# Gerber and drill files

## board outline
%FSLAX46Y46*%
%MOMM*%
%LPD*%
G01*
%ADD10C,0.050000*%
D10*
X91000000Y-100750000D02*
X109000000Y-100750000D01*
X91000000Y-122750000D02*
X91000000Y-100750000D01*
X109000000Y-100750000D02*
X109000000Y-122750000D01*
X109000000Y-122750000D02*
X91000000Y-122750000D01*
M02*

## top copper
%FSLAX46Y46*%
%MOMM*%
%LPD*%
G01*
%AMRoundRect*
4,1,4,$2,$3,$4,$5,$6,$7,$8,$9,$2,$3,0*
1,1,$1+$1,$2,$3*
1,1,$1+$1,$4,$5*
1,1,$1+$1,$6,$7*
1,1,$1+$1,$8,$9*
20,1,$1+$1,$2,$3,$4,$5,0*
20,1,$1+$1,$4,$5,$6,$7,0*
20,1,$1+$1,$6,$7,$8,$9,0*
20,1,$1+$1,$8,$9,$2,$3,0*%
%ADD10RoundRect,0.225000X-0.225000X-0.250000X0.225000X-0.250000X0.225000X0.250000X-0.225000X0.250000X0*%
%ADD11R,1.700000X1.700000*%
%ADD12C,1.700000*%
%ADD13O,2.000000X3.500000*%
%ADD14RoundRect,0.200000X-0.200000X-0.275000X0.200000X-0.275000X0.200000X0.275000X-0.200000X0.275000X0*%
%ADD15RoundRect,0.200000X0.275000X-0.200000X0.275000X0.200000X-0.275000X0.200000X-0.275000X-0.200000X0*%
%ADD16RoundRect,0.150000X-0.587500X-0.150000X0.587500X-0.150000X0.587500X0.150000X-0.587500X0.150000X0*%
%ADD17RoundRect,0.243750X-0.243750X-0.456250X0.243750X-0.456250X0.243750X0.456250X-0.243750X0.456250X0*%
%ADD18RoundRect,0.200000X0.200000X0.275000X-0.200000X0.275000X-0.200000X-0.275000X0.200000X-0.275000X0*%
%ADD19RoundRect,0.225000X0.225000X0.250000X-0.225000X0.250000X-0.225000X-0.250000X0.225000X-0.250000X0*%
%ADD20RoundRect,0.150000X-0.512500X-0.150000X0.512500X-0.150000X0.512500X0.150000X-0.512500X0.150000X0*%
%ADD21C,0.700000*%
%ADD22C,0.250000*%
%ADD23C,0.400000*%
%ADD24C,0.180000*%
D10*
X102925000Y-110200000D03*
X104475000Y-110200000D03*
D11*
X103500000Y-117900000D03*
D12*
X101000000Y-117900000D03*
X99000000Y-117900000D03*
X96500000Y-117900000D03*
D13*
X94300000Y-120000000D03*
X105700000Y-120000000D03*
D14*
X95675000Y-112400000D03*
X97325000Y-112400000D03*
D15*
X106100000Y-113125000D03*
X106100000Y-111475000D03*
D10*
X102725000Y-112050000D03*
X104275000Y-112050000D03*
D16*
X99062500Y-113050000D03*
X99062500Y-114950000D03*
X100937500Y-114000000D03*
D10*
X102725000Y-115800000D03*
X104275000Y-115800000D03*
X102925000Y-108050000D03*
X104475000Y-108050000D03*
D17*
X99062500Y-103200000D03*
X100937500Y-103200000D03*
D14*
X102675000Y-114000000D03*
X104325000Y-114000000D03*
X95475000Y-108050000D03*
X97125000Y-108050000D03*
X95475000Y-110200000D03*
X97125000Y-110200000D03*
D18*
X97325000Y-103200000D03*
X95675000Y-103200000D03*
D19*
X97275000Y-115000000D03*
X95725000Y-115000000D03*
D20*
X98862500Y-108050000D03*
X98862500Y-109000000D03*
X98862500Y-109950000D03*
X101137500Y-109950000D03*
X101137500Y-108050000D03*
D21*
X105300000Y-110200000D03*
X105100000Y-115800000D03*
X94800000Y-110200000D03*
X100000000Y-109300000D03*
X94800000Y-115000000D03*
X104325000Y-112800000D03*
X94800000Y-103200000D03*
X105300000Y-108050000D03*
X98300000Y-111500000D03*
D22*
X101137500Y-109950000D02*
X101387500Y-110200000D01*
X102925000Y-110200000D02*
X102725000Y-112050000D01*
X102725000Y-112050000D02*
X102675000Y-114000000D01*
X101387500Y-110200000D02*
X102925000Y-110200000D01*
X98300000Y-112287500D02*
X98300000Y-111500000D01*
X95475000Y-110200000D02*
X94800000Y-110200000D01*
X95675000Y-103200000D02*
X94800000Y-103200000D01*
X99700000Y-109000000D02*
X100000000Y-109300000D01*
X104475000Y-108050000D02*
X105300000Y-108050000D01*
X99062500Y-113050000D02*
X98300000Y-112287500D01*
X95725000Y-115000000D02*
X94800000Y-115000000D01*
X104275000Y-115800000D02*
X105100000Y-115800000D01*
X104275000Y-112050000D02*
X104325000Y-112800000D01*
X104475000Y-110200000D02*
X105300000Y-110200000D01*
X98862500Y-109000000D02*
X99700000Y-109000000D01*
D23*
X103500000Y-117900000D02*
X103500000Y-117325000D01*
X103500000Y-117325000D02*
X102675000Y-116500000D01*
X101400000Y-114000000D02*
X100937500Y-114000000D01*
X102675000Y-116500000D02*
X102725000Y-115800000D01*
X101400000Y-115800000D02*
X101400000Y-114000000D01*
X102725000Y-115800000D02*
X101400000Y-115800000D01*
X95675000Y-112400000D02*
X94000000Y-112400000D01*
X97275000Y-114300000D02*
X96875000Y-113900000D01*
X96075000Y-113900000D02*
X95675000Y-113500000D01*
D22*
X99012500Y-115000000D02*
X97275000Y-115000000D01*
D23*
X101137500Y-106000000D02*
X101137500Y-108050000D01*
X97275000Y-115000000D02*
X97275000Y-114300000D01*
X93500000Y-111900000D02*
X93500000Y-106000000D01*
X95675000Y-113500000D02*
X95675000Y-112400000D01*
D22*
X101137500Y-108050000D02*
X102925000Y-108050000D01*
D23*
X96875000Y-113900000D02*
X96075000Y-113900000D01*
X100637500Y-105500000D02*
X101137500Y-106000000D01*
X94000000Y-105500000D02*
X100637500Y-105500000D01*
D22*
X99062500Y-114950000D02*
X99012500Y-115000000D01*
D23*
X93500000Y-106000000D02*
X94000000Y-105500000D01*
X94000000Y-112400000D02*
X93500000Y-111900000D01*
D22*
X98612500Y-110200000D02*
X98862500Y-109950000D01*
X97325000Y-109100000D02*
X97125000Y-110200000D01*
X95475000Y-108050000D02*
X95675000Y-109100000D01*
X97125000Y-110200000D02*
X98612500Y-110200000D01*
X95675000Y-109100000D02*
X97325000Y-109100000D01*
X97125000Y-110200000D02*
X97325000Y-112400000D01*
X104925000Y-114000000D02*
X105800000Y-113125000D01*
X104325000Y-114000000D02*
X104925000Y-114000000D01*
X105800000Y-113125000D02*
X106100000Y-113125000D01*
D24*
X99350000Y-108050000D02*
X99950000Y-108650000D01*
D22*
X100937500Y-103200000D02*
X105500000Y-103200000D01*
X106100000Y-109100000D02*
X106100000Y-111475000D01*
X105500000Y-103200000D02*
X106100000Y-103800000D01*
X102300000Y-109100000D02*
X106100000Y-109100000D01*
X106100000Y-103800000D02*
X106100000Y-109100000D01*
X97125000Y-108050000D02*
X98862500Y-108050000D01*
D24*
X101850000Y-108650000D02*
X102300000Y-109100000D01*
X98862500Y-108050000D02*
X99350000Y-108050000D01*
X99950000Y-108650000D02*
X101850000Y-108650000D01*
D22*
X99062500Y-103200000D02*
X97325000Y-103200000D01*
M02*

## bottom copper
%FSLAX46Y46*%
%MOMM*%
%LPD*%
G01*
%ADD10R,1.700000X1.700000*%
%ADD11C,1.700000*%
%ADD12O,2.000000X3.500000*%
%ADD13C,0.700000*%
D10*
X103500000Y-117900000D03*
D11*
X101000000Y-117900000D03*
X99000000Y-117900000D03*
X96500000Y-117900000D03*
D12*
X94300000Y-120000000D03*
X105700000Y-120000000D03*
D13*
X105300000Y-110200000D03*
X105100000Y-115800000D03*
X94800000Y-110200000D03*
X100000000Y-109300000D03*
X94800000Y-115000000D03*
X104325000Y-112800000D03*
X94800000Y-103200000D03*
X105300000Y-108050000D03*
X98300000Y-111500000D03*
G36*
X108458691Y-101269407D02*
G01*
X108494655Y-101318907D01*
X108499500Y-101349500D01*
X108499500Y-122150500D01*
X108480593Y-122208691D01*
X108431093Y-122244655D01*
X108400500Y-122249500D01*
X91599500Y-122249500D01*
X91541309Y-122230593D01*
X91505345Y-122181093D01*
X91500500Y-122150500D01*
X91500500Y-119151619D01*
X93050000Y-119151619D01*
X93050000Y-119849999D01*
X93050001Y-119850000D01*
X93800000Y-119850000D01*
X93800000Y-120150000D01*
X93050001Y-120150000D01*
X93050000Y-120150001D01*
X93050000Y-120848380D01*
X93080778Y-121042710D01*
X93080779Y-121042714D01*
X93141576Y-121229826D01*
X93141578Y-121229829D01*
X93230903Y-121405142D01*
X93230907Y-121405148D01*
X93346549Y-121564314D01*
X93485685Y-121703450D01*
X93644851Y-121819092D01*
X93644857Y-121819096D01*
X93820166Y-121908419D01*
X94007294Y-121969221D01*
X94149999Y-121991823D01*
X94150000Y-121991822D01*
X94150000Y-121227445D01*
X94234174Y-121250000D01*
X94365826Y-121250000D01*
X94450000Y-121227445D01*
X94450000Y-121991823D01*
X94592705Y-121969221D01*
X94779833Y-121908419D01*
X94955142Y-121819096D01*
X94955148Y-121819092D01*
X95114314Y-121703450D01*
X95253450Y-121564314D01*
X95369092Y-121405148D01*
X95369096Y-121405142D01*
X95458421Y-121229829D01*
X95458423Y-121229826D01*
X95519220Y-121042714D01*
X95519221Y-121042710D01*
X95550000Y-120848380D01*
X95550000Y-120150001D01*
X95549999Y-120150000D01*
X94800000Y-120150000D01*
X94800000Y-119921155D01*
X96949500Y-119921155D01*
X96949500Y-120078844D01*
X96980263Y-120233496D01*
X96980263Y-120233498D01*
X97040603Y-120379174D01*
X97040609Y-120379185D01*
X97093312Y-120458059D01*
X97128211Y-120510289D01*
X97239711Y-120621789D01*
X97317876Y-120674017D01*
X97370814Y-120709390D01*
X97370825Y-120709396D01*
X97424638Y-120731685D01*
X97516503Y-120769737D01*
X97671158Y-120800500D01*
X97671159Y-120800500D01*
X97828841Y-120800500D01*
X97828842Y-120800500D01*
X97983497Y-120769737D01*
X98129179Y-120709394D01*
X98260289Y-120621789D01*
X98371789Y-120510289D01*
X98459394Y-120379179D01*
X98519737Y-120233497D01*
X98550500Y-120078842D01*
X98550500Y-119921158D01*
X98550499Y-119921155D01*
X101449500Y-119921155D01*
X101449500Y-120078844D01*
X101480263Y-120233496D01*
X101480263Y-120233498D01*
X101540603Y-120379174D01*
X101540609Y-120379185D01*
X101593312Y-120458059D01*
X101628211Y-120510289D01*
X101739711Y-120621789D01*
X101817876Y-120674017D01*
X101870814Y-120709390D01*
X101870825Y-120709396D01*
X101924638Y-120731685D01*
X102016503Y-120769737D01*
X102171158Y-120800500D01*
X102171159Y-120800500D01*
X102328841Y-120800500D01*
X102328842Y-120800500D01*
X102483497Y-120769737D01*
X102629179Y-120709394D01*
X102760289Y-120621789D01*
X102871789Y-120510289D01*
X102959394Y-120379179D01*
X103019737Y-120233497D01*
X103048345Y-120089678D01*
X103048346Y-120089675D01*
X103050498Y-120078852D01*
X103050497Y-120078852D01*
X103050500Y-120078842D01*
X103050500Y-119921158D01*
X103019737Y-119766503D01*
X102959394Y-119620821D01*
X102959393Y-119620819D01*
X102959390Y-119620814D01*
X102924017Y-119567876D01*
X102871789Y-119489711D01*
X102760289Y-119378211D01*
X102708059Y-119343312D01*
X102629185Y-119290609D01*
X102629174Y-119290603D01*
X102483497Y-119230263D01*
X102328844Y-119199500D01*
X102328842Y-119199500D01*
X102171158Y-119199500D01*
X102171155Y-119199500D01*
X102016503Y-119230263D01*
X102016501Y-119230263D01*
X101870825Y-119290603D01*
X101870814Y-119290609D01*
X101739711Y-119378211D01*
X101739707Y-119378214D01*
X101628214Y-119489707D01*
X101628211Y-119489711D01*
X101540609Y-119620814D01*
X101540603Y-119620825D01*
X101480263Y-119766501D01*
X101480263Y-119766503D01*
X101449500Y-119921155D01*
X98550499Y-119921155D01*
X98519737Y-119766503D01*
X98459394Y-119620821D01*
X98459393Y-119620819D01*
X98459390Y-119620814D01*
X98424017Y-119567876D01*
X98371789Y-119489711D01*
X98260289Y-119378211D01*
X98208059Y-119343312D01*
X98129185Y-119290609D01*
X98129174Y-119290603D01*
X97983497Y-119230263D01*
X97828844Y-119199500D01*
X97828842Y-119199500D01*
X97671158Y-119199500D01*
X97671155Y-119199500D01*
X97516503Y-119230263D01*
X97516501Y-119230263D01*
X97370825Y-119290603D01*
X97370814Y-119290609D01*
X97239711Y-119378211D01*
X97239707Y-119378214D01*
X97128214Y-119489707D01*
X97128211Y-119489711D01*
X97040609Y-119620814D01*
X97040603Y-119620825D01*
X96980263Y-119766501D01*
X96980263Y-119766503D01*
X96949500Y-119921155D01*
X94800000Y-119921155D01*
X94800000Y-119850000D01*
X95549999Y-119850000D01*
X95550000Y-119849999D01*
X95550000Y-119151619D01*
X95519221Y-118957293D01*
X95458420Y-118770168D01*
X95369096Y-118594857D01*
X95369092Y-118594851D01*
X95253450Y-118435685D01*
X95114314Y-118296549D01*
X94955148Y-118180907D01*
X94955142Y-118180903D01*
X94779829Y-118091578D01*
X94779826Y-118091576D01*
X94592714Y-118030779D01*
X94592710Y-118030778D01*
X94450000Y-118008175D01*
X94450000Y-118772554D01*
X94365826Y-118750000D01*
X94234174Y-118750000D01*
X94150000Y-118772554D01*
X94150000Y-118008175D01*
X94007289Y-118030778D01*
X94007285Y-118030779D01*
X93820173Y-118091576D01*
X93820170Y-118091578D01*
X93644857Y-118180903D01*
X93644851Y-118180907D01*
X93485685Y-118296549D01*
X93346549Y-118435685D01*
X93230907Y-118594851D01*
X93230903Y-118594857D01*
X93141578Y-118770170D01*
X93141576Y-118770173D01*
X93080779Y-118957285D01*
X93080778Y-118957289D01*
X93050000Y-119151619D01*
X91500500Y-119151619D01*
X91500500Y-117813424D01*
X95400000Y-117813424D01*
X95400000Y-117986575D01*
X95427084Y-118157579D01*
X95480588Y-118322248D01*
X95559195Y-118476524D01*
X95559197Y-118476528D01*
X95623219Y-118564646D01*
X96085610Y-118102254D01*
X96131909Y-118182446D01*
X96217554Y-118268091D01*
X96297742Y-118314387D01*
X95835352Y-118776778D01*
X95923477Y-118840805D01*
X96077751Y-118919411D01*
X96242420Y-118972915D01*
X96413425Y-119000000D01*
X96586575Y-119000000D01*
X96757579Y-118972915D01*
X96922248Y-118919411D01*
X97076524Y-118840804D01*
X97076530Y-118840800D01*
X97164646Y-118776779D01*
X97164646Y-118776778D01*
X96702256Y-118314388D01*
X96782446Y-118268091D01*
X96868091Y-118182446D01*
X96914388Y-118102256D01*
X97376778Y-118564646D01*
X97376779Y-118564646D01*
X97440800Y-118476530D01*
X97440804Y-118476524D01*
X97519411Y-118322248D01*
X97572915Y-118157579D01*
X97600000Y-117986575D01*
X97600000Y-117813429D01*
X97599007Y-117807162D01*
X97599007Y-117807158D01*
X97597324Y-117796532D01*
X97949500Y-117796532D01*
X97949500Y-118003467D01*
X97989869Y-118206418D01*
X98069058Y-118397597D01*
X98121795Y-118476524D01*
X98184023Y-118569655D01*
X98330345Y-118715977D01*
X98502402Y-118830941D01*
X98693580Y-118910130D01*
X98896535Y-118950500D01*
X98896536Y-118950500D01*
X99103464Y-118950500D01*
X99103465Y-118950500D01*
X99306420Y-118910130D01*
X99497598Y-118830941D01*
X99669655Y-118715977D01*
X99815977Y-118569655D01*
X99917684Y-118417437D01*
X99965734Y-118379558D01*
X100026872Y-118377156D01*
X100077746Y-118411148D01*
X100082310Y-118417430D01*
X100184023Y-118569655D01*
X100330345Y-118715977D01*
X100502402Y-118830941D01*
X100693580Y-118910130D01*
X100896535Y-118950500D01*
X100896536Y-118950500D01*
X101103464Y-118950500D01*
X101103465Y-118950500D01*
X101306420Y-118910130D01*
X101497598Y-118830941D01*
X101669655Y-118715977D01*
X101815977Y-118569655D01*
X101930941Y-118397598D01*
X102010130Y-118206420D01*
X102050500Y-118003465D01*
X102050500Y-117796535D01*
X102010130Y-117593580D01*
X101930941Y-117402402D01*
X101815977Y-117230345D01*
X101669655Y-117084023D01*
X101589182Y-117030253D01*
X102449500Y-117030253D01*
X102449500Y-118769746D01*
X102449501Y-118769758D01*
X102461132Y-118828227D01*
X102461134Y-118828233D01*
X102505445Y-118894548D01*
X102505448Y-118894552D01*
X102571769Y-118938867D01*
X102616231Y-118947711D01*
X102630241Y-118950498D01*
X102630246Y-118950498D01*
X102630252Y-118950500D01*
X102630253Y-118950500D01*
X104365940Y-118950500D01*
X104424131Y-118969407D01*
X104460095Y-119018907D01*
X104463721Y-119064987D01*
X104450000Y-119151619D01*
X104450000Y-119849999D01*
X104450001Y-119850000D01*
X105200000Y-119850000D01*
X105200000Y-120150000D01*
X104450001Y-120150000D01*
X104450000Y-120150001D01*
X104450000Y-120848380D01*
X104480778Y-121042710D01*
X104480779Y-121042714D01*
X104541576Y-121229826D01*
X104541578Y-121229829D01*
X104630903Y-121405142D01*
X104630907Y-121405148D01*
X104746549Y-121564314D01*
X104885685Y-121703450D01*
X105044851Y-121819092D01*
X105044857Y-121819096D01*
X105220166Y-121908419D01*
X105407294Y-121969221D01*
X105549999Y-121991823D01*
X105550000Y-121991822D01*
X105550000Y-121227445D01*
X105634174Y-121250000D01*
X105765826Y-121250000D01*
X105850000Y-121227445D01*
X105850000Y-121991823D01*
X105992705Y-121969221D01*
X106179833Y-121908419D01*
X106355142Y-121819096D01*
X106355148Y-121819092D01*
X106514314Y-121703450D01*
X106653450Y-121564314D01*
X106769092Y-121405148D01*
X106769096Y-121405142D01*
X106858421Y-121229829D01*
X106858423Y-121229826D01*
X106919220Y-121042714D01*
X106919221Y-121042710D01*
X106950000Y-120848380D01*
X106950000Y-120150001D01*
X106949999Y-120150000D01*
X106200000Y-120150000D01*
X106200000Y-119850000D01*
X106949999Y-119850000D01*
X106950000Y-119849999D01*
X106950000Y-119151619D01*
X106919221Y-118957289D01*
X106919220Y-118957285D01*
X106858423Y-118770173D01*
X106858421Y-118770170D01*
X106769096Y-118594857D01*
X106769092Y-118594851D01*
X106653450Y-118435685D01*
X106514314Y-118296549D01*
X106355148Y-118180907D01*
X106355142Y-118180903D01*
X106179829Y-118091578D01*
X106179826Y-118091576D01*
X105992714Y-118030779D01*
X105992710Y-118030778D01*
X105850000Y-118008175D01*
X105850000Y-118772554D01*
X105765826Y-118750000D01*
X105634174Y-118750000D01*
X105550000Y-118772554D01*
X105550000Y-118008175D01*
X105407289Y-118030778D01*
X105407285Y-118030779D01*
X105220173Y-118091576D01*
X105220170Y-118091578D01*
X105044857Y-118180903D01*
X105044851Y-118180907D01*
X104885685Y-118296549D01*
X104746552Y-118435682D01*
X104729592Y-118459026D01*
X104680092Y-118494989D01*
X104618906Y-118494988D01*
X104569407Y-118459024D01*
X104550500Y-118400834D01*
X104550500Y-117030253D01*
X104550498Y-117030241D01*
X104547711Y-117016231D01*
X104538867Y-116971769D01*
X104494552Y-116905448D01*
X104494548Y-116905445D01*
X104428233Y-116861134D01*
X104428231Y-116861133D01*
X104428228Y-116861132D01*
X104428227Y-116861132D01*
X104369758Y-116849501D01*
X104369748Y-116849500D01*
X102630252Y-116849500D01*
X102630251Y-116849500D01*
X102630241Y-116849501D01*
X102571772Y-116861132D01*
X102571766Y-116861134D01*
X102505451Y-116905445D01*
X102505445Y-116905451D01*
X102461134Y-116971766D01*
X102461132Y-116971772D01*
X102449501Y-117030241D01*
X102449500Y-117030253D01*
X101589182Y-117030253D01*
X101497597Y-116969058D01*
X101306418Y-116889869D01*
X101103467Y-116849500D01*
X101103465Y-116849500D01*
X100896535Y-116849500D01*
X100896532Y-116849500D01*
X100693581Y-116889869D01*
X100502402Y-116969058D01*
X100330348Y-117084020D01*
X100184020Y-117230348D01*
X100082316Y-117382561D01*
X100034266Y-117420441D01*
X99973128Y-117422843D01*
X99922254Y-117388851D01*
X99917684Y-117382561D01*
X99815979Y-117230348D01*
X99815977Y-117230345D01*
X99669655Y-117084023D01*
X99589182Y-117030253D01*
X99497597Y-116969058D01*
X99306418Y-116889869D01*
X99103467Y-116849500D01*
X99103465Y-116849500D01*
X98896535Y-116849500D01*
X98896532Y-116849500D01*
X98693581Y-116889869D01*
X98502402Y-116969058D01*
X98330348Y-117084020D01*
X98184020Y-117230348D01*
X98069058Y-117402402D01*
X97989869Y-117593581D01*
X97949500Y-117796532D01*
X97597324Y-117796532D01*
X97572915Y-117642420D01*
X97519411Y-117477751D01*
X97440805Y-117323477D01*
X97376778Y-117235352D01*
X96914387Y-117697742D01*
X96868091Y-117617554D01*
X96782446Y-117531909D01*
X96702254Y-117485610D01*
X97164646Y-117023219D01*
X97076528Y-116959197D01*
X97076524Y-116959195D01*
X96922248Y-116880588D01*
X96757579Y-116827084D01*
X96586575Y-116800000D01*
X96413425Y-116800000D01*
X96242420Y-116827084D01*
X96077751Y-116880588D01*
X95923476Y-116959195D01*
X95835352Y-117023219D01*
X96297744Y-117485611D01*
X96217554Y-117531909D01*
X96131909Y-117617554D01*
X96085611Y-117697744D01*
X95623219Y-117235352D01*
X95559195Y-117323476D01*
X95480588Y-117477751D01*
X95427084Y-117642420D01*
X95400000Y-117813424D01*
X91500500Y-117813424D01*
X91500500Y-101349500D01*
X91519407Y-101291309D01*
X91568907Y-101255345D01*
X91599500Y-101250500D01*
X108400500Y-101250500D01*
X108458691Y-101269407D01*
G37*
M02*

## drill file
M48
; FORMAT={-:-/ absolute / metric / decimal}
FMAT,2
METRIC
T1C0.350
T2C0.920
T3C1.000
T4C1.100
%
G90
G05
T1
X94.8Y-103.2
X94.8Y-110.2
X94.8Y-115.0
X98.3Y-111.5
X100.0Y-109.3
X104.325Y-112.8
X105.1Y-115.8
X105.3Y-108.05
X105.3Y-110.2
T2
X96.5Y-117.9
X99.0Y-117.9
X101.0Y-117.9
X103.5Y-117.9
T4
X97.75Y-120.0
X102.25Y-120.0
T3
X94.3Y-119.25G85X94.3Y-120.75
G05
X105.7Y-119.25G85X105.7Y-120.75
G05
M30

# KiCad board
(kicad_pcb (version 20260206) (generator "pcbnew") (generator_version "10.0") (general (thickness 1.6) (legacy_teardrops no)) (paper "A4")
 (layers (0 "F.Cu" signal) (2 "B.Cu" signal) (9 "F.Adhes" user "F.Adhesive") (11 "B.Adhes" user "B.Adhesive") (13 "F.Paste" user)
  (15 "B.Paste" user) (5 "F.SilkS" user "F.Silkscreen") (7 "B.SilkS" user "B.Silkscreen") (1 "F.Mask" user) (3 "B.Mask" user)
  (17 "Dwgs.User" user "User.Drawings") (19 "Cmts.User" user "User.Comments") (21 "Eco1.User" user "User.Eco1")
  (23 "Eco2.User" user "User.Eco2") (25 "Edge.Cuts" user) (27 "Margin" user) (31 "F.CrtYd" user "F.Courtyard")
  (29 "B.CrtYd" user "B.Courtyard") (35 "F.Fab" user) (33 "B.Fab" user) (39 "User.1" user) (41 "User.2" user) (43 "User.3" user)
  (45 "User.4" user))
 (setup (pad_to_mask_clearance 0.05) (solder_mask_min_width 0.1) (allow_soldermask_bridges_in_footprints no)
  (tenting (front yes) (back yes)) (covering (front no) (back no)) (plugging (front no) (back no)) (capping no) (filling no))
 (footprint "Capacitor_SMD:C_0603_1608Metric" (layer "F.Cu") (at 103.7 110.2)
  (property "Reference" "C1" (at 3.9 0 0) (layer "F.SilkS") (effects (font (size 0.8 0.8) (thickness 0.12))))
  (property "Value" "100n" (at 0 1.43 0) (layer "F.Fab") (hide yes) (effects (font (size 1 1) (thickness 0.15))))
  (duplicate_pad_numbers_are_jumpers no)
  (pad "1" smd roundrect (at -0.775 0) (size 0.9 0.95) (layers "F.Cu" "F.Mask" "F.Paste") (roundrect_rratio 0.25) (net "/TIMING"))
  (pad "2" smd roundrect (at 0.775 0) (size 0.9 0.95) (layers "F.Cu" "F.Mask" "F.Paste") (roundrect_rratio 0.25) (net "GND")))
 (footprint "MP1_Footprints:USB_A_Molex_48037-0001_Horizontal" (layer "F.Cu") (at 100 120)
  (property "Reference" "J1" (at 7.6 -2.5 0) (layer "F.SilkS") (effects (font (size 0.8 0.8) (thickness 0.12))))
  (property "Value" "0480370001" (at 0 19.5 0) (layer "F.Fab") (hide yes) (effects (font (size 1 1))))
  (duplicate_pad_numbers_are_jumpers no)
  (pad "" np_thru_hole circle (at -2.25 0) (size 1.1 1.1) (drill 1.1) (layers "*.Mask"))
  (pad "" np_thru_hole circle (at 2.25 0) (size 1.1 1.1) (drill 1.1) (layers "*.Mask"))
  (pad "1" thru_hole rect (at 3.5 -2.1) (size 1.7 1.7) (drill 0.92) (layers "*.Cu" "*.Mask") (remove_unused_layers no) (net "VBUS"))
  (pad "2" thru_hole circle (at 1 -2.1) (size 1.7 1.7) (drill 0.92) (layers "*.Cu" "*.Mask") (remove_unused_layers no)
   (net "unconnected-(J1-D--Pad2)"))
  (pad "3" thru_hole circle (at -1 -2.1) (size 1.7 1.7) (drill 0.92) (layers "*.Cu" "*.Mask") (remove_unused_layers no)
   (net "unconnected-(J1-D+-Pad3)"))
  (pad "4" thru_hole circle (at -3.5 -2.1) (size 1.7 1.7) (drill 0.92) (layers "*.Cu" "*.Mask") (remove_unused_layers no) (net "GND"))
  (pad "SH" thru_hole oval (at -5.7 0) (size 2 3.5) (drill oval 1 2.5) (layers "*.Cu" "*.Mask") (remove_unused_layers no) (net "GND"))
  (pad "SH" thru_hole oval (at 5.7 0) (size 2 3.5) (drill oval 1 2.5) (layers "*.Cu" "*.Mask") (remove_unused_layers no) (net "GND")))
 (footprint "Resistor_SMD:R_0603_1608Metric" (layer "F.Cu") (at 96.5 112.4)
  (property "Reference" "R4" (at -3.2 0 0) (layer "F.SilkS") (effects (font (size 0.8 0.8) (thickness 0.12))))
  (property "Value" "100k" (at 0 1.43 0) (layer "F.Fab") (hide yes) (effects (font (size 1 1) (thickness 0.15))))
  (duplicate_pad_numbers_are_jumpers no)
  (pad "1" smd roundrect (at -0.825 0) (size 0.8 0.95) (layers "F.Cu" "F.Mask" "F.Paste") (roundrect_rratio 0.25) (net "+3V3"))
  (pad "2" smd roundrect (at 0.825 0) (size 0.8 0.95) (layers "F.Cu" "F.Mask" "F.Paste") (roundrect_rratio 0.25) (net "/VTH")))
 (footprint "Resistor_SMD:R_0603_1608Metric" (layer "F.Cu") (at 106.1 112.3 90)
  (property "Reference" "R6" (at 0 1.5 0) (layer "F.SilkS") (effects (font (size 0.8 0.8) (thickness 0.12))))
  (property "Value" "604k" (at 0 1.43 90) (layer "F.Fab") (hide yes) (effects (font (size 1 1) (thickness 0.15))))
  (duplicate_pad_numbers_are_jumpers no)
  (pad "1" smd roundrect (at -0.825 0 90) (size 0.8 0.95) (layers "F.Cu" "F.Mask" "F.Paste") (roundrect_rratio 0.25) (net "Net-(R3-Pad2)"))
  (pad "2" smd roundrect (at 0.825 0 90) (size 0.8 0.95) (layers "F.Cu" "F.Mask" "F.Paste") (roundrect_rratio 0.25) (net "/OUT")))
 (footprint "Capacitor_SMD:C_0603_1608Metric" (layer "F.Cu") (at 103.5 112.05)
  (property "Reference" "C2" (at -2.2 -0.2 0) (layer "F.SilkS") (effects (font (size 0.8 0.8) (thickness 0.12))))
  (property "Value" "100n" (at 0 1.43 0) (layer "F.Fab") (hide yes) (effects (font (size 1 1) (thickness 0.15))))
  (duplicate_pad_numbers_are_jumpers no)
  (pad "1" smd roundrect (at -0.775 0) (size 0.9 0.95) (layers "F.Cu" "F.Mask" "F.Paste") (roundrect_rratio 0.25) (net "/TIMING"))
  (pad "2" smd roundrect (at 0.775 0) (size 0.9 0.95) (layers "F.Cu" "F.Mask" "F.Paste") (roundrect_rratio 0.25) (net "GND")))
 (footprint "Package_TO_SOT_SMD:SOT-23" (layer "F.Cu") (at 100 114)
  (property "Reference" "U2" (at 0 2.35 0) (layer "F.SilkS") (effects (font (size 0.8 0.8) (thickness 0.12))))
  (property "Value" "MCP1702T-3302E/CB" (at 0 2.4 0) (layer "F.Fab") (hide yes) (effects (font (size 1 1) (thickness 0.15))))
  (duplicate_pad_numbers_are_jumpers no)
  (pad "1" smd roundrect (at -0.9375 -0.95) (size 1.475 0.6) (layers "F.Cu" "F.Mask" "F.Paste") (roundrect_rratio 0.25) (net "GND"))
  (pad "2" smd roundrect (at -0.9375 0.95) (size 1.475 0.6) (layers "F.Cu" "F.Mask" "F.Paste") (roundrect_rratio 0.25) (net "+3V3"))
  (pad "3" smd roundrect (at 0.9375 0) (size 1.475 0.6) (layers "F.Cu" "F.Mask" "F.Paste") (roundrect_rratio 0.25) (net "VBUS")))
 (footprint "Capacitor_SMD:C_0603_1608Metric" (layer "F.Cu") (at 103.5 115.8)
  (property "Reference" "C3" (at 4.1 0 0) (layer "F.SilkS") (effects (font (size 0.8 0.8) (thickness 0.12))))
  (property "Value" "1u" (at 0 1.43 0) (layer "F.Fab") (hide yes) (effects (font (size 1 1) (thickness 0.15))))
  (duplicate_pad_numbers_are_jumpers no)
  (pad "1" smd roundrect (at -0.775 0) (size 0.9 0.95) (layers "F.Cu" "F.Mask" "F.Paste") (roundrect_rratio 0.25) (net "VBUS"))
  (pad "2" smd roundrect (at 0.775 0) (size 0.9 0.95) (layers "F.Cu" "F.Mask" "F.Paste") (roundrect_rratio 0.25) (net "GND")))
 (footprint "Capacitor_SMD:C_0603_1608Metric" (layer "F.Cu") (at 103.7 108.05)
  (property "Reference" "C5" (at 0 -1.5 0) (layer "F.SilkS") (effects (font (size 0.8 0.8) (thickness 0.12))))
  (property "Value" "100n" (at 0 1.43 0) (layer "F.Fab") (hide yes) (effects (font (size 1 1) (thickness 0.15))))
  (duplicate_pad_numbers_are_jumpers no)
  (pad "1" smd roundrect (at -0.775 0) (size 0.9 0.95) (layers "F.Cu" "F.Mask" "F.Paste") (roundrect_rratio 0.25) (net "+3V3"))
  (pad "2" smd roundrect (at 0.775 0) (size 0.9 0.95) (layers "F.Cu" "F.Mask" "F.Paste") (roundrect_rratio 0.25) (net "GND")))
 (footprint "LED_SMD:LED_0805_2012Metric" (layer "F.Cu") (at 100 103.2)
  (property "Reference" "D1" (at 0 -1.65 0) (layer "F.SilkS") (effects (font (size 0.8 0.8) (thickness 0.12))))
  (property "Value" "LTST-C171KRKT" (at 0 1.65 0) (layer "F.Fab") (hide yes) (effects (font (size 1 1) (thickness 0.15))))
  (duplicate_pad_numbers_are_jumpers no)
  (pad "1" smd roundrect (at -0.9375 0) (size 0.975 1.4) (layers "F.Cu" "F.Mask" "F.Paste") (roundrect_rratio 0.25) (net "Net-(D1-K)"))
  (pad "2" smd roundrect (at 0.9375 0) (size 0.975 1.4) (layers "F.Cu" "F.Mask" "F.Paste") (roundrect_rratio 0.25) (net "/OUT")))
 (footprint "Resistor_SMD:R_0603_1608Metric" (layer "F.Cu") (at 103.5 114)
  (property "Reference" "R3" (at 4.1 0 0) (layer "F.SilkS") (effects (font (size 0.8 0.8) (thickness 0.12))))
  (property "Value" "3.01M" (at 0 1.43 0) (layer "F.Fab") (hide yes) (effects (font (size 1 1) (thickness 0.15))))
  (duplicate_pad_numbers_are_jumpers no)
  (pad "1" smd roundrect (at -0.825 0) (size 0.8 0.95) (layers "F.Cu" "F.Mask" "F.Paste") (roundrect_rratio 0.25) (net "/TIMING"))
  (pad "2" smd roundrect (at 0.825 0) (size 0.8 0.95) (layers "F.Cu" "F.Mask" "F.Paste") (roundrect_rratio 0.25) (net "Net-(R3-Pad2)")))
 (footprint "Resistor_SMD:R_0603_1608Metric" (layer "F.Cu") (at 96.3 108.05)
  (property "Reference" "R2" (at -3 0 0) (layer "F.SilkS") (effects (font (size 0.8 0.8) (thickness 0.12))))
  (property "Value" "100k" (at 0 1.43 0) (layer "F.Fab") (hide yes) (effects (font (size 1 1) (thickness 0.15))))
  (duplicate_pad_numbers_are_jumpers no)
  (pad "1" smd roundrect (at -0.825 0) (size 0.8 0.95) (layers "F.Cu" "F.Mask" "F.Paste") (roundrect_rratio 0.25) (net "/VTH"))
  (pad "2" smd roundrect (at 0.825 0) (size 0.8 0.95) (layers "F.Cu" "F.Mask" "F.Paste") (roundrect_rratio 0.25) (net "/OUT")))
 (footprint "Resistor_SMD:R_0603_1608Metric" (layer "F.Cu") (at 96.3 110.2)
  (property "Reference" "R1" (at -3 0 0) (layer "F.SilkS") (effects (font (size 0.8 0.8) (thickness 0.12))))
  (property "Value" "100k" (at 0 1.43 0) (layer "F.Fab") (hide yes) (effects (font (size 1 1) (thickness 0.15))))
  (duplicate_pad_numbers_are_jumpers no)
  (pad "1" smd roundrect (at -0.825 0) (size 0.8 0.95) (layers "F.Cu" "F.Mask" "F.Paste") (roundrect_rratio 0.25) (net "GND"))
  (pad "2" smd roundrect (at 0.825 0) (size 0.8 0.95) (layers "F.Cu" "F.Mask" "F.Paste") (roundrect_rratio 0.25) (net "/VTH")))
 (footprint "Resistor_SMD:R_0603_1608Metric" (layer "F.Cu") (at 96.5 103.2 180)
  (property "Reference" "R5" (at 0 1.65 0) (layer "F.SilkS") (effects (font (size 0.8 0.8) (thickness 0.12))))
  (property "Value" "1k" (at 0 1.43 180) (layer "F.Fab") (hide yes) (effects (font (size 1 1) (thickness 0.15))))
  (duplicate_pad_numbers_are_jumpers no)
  (pad "1" smd roundrect (at -0.825 0 180) (size 0.8 0.95) (layers "F.Cu" "F.Mask" "F.Paste") (roundrect_rratio 0.25) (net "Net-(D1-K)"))
  (pad "2" smd roundrect (at 0.825 0 180) (size 0.8 0.95) (layers "F.Cu" "F.Mask" "F.Paste") (roundrect_rratio 0.25) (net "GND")))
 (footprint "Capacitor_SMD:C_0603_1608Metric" (layer "F.Cu") (at 96.5 115 180)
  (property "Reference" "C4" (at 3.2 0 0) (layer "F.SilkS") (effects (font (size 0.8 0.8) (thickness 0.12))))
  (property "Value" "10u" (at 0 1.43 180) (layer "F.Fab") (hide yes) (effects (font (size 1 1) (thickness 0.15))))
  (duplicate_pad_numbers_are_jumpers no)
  (pad "1" smd roundrect (at -0.775 0 180) (size 0.9 0.95) (layers "F.Cu" "F.Mask" "F.Paste") (roundrect_rratio 0.25) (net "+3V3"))
  (pad "2" smd roundrect (at 0.775 0 180) (size 0.9 0.95) (layers "F.Cu" "F.Mask" "F.Paste") (roundrect_rratio 0.25) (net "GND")))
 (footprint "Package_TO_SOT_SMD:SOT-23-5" (layer "F.Cu") (at 100 109)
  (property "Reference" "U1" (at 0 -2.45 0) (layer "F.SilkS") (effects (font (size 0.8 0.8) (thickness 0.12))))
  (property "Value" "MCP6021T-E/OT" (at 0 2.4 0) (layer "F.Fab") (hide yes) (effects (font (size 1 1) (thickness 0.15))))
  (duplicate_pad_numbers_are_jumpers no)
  (pad "1" smd roundrect (at -1.1375 -0.95) (size 1.325 0.6) (layers "F.Cu" "F.Mask" "F.Paste") (roundrect_rratio 0.25) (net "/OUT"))
  (pad "2" smd roundrect (at -1.1375 0) (size 1.325 0.6) (layers "F.Cu" "F.Mask" "F.Paste") (roundrect_rratio 0.25) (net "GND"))
  (pad "3" smd roundrect (at -1.1375 0.95) (size 1.325 0.6) (layers "F.Cu" "F.Mask" "F.Paste") (roundrect_rratio 0.25) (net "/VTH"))
  (pad "4" smd roundrect (at 1.1375 0.95) (size 1.325 0.6) (layers "F.Cu" "F.Mask" "F.Paste") (roundrect_rratio 0.25) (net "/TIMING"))
  (pad "5" smd roundrect (at 1.1375 -0.95) (size 1.325 0.6) (layers "F.Cu" "F.Mask" "F.Paste") (roundrect_rratio 0.25) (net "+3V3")))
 (gr_line (start 91 100.75) (end 109 100.75) (stroke (width 0.05) (type default)) (layer "Edge.Cuts"))
 (gr_line (start 91 122.75) (end 91 100.75) (stroke (width 0.05) (type default)) (layer "Edge.Cuts"))
 (gr_line (start 109 100.75) (end 109 122.75) (stroke (width 0.05) (type default)) (layer "Edge.Cuts"))
 (gr_line (start 109 122.75) (end 91 122.75) (stroke (width 0.05) (type default)) (layer "Edge.Cuts"))
 (segment (start 101.1375 109.95) (end 101.3875 110.2) (width 0.25) (layer "F.Cu") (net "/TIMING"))
 (segment (start 102.925 110.2) (end 102.725 112.05) (width 0.25) (layer "F.Cu") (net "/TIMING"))
 (segment (start 102.725 112.05) (end 102.675 114) (width 0.25) (layer "F.Cu") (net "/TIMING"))
 (segment (start 101.3875 110.2) (end 102.925 110.2) (width 0.25) (layer "F.Cu") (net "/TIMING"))
 (segment (start 98.3 112.2875) (end 98.3 111.5) (width 0.25) (layer "F.Cu") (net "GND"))
 (segment (start 95.475 110.2) (end 94.8 110.2) (width 0.25) (layer "F.Cu") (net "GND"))
 (segment (start 95.675 103.2) (end 94.8 103.2) (width 0.25) (layer "F.Cu") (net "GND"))
 (segment (start 99.7 109) (end 100 109.3) (width 0.25) (layer "F.Cu") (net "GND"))
 (segment (start 104.475 108.05) (end 105.3 108.05) (width 0.25) (layer "F.Cu") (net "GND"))
 (segment (start 99.0625 113.05) (end 98.3 112.2875) (width 0.25) (layer "F.Cu") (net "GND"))
 (segment (start 95.725 115) (end 94.8 115) (width 0.25) (layer "F.Cu") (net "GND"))
 (segment (start 104.275 115.8) (end 105.1 115.8) (width 0.25) (layer "F.Cu") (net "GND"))
 (segment (start 104.275 112.05) (end 104.325 112.8) (width 0.25) (layer "F.Cu") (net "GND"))
 (segment (start 104.475 110.2) (end 105.3 110.2) (width 0.25) (layer "F.Cu") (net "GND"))
 (segment (start 98.8625 109) (end 99.7 109) (width 0.25) (layer "F.Cu") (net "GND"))
 (via (at 105.3 110.2) (size 0.7) (drill 0.35) (layers "F.Cu" "B.Cu") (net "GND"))
 (via (at 105.1 115.8) (size 0.7) (drill 0.35) (layers "F.Cu" "B.Cu") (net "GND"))
 (via (at 94.8 110.2) (size 0.7) (drill 0.35) (layers "F.Cu" "B.Cu") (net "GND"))
 (via (at 100 109.3) (size 0.7) (drill 0.35) (layers "F.Cu" "B.Cu") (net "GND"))
 (via (at 94.8 115) (size 0.7) (drill 0.35) (layers "F.Cu" "B.Cu") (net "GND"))
 (via (at 104.325 112.8) (size 0.7) (drill 0.35) (layers "F.Cu" "B.Cu") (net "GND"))
 (via (at 94.8 103.2) (size 0.7) (drill 0.35) (layers "F.Cu" "B.Cu") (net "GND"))
 (via (at 105.3 108.05) (size 0.7) (drill 0.35) (layers "F.Cu" "B.Cu") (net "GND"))
 (via (at 98.3 111.5) (size 0.7) (drill 0.35) (layers "F.Cu" "B.Cu") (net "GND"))
 (segment (start 103.5 117.9) (end 103.5 117.325) (width 0.4) (layer "F.Cu") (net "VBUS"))
 (segment (start 103.5 117.325) (end 102.675 116.5) (width 0.4) (layer "F.Cu") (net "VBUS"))
 (segment (start 101.4 114) (end 100.9375 114) (width 0.4) (layer "F.Cu") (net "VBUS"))
 (segment (start 102.675 116.5) (end 102.725 115.8) (width 0.4) (layer "F.Cu") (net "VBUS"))
 (segment (start 101.4 115.8) (end 101.4 114) (width 0.4) (layer "F.Cu") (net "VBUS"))
 (segment (start 102.725 115.8) (end 101.4 115.8) (width 0.4) (layer "F.Cu") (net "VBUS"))
 (segment (start 95.675 112.4) (end 94 112.4) (width 0.4) (layer "F.Cu") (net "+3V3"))
 (segment (start 97.275 114.3) (end 96.875 113.9) (width 0.4) (layer "F.Cu") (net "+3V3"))
 (segment (start 96.075 113.9) (end 95.675 113.5) (width 0.4) (layer "F.Cu") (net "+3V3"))
 (segment (start 99.0125 115) (end 97.275 115) (width 0.25) (layer "F.Cu") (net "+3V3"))
 (segment (start 101.1375 106) (end 101.1375 108.05) (width 0.4) (layer "F.Cu") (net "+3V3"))
 (segment (start 97.275 115) (end 97.275 114.3) (width 0.4) (layer "F.Cu") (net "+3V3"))
 (segment (start 93.5 111.9) (end 93.5 106) (width 0.4) (layer "F.Cu") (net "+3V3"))
 (segment (start 95.675 113.5) (end 95.675 112.4) (width 0.4) (layer "F.Cu") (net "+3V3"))
 (segment (start 101.1375 108.05) (end 102.925 108.05) (width 0.25) (layer "F.Cu") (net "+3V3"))
 (segment (start 96.875 113.9) (end 96.075 113.9) (width 0.4) (layer "F.Cu") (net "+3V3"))
 (segment (start 100.6375 105.5) (end 101.1375 106) (width 0.4) (layer "F.Cu") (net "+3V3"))
 (segment (start 94 105.5) (end 100.6375 105.5) (width 0.4) (layer "F.Cu") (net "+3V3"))
 (segment (start 99.0625 114.95) (end 99.0125 115) (width 0.25) (layer "F.Cu") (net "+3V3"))
 (segment (start 93.5 106) (end 94 105.5) (width 0.4) (layer "F.Cu") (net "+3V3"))
 (segment (start 94 112.4) (end 93.5 111.9) (width 0.4) (layer "F.Cu") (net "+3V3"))
 (segment (start 98.6125 110.2) (end 98.8625 109.95) (width 0.25) (layer "F.Cu") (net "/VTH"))
 (segment (start 97.325 109.1) (end 97.125 110.2) (width 0.25) (layer "F.Cu") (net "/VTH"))
 (segment (start 95.475 108.05) (end 95.675 109.1) (width 0.25) (layer "F.Cu") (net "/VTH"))
 (segment (start 97.125 110.2) (end 98.6125 110.2) (width 0.25) (layer "F.Cu") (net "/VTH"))
 (segment (start 95.675 109.1) (end 97.325 109.1) (width 0.25) (layer "F.Cu") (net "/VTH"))
 (segment (start 97.125 110.2) (end 97.325 112.4) (width 0.25) (layer "F.Cu") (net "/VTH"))
 (segment (start 104.925 114) (end 105.8 113.125) (width 0.25) (layer "F.Cu") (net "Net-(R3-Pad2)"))
 (segment (start 104.325 114) (end 104.925 114) (width 0.25) (layer "F.Cu") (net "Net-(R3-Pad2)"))
 (segment (start 105.8 113.125) (end 106.1 113.125) (width 0.25) (layer "F.Cu") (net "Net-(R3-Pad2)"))
 (segment (start 99.35 108.05) (end 99.95 108.65) (width 0.18) (layer "F.Cu") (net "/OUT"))
 (segment (start 100.9375 103.2) (end 105.5 103.2) (width 0.25) (layer "F.Cu") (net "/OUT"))
 (segment (start 106.1 109.1) (end 106.1 111.475) (width 0.25) (layer "F.Cu") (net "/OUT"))
 (segment (start 105.5 103.2) (end 106.1 103.8) (width 0.25) (layer "F.Cu") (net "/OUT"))
 (segment (start 102.3 109.1) (end 106.1 109.1) (width 0.25) (layer "F.Cu") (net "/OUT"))
 (segment (start 106.1 103.8) (end 106.1 109.1) (width 0.25) (layer "F.Cu") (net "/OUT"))
 (segment (start 97.125 108.05) (end 98.8625 108.05) (width 0.25) (layer "F.Cu") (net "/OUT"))
 (segment (start 101.85 108.65) (end 102.3 109.1) (width 0.18) (layer "F.Cu") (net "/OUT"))
 (segment (start 98.8625 108.05) (end 99.35 108.05) (width 0.18) (layer "F.Cu") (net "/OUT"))
 (segment (start 99.95 108.65) (end 101.85 108.65) (width 0.18) (layer "F.Cu") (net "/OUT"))
 (segment (start 99.0625 103.2) (end 97.325 103.2) (width 0.25) (layer "F.Cu") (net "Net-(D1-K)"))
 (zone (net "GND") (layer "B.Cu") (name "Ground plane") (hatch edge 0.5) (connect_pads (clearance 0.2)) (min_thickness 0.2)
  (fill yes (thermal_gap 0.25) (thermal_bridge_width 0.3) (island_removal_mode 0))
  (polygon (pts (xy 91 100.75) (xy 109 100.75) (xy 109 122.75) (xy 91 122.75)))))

